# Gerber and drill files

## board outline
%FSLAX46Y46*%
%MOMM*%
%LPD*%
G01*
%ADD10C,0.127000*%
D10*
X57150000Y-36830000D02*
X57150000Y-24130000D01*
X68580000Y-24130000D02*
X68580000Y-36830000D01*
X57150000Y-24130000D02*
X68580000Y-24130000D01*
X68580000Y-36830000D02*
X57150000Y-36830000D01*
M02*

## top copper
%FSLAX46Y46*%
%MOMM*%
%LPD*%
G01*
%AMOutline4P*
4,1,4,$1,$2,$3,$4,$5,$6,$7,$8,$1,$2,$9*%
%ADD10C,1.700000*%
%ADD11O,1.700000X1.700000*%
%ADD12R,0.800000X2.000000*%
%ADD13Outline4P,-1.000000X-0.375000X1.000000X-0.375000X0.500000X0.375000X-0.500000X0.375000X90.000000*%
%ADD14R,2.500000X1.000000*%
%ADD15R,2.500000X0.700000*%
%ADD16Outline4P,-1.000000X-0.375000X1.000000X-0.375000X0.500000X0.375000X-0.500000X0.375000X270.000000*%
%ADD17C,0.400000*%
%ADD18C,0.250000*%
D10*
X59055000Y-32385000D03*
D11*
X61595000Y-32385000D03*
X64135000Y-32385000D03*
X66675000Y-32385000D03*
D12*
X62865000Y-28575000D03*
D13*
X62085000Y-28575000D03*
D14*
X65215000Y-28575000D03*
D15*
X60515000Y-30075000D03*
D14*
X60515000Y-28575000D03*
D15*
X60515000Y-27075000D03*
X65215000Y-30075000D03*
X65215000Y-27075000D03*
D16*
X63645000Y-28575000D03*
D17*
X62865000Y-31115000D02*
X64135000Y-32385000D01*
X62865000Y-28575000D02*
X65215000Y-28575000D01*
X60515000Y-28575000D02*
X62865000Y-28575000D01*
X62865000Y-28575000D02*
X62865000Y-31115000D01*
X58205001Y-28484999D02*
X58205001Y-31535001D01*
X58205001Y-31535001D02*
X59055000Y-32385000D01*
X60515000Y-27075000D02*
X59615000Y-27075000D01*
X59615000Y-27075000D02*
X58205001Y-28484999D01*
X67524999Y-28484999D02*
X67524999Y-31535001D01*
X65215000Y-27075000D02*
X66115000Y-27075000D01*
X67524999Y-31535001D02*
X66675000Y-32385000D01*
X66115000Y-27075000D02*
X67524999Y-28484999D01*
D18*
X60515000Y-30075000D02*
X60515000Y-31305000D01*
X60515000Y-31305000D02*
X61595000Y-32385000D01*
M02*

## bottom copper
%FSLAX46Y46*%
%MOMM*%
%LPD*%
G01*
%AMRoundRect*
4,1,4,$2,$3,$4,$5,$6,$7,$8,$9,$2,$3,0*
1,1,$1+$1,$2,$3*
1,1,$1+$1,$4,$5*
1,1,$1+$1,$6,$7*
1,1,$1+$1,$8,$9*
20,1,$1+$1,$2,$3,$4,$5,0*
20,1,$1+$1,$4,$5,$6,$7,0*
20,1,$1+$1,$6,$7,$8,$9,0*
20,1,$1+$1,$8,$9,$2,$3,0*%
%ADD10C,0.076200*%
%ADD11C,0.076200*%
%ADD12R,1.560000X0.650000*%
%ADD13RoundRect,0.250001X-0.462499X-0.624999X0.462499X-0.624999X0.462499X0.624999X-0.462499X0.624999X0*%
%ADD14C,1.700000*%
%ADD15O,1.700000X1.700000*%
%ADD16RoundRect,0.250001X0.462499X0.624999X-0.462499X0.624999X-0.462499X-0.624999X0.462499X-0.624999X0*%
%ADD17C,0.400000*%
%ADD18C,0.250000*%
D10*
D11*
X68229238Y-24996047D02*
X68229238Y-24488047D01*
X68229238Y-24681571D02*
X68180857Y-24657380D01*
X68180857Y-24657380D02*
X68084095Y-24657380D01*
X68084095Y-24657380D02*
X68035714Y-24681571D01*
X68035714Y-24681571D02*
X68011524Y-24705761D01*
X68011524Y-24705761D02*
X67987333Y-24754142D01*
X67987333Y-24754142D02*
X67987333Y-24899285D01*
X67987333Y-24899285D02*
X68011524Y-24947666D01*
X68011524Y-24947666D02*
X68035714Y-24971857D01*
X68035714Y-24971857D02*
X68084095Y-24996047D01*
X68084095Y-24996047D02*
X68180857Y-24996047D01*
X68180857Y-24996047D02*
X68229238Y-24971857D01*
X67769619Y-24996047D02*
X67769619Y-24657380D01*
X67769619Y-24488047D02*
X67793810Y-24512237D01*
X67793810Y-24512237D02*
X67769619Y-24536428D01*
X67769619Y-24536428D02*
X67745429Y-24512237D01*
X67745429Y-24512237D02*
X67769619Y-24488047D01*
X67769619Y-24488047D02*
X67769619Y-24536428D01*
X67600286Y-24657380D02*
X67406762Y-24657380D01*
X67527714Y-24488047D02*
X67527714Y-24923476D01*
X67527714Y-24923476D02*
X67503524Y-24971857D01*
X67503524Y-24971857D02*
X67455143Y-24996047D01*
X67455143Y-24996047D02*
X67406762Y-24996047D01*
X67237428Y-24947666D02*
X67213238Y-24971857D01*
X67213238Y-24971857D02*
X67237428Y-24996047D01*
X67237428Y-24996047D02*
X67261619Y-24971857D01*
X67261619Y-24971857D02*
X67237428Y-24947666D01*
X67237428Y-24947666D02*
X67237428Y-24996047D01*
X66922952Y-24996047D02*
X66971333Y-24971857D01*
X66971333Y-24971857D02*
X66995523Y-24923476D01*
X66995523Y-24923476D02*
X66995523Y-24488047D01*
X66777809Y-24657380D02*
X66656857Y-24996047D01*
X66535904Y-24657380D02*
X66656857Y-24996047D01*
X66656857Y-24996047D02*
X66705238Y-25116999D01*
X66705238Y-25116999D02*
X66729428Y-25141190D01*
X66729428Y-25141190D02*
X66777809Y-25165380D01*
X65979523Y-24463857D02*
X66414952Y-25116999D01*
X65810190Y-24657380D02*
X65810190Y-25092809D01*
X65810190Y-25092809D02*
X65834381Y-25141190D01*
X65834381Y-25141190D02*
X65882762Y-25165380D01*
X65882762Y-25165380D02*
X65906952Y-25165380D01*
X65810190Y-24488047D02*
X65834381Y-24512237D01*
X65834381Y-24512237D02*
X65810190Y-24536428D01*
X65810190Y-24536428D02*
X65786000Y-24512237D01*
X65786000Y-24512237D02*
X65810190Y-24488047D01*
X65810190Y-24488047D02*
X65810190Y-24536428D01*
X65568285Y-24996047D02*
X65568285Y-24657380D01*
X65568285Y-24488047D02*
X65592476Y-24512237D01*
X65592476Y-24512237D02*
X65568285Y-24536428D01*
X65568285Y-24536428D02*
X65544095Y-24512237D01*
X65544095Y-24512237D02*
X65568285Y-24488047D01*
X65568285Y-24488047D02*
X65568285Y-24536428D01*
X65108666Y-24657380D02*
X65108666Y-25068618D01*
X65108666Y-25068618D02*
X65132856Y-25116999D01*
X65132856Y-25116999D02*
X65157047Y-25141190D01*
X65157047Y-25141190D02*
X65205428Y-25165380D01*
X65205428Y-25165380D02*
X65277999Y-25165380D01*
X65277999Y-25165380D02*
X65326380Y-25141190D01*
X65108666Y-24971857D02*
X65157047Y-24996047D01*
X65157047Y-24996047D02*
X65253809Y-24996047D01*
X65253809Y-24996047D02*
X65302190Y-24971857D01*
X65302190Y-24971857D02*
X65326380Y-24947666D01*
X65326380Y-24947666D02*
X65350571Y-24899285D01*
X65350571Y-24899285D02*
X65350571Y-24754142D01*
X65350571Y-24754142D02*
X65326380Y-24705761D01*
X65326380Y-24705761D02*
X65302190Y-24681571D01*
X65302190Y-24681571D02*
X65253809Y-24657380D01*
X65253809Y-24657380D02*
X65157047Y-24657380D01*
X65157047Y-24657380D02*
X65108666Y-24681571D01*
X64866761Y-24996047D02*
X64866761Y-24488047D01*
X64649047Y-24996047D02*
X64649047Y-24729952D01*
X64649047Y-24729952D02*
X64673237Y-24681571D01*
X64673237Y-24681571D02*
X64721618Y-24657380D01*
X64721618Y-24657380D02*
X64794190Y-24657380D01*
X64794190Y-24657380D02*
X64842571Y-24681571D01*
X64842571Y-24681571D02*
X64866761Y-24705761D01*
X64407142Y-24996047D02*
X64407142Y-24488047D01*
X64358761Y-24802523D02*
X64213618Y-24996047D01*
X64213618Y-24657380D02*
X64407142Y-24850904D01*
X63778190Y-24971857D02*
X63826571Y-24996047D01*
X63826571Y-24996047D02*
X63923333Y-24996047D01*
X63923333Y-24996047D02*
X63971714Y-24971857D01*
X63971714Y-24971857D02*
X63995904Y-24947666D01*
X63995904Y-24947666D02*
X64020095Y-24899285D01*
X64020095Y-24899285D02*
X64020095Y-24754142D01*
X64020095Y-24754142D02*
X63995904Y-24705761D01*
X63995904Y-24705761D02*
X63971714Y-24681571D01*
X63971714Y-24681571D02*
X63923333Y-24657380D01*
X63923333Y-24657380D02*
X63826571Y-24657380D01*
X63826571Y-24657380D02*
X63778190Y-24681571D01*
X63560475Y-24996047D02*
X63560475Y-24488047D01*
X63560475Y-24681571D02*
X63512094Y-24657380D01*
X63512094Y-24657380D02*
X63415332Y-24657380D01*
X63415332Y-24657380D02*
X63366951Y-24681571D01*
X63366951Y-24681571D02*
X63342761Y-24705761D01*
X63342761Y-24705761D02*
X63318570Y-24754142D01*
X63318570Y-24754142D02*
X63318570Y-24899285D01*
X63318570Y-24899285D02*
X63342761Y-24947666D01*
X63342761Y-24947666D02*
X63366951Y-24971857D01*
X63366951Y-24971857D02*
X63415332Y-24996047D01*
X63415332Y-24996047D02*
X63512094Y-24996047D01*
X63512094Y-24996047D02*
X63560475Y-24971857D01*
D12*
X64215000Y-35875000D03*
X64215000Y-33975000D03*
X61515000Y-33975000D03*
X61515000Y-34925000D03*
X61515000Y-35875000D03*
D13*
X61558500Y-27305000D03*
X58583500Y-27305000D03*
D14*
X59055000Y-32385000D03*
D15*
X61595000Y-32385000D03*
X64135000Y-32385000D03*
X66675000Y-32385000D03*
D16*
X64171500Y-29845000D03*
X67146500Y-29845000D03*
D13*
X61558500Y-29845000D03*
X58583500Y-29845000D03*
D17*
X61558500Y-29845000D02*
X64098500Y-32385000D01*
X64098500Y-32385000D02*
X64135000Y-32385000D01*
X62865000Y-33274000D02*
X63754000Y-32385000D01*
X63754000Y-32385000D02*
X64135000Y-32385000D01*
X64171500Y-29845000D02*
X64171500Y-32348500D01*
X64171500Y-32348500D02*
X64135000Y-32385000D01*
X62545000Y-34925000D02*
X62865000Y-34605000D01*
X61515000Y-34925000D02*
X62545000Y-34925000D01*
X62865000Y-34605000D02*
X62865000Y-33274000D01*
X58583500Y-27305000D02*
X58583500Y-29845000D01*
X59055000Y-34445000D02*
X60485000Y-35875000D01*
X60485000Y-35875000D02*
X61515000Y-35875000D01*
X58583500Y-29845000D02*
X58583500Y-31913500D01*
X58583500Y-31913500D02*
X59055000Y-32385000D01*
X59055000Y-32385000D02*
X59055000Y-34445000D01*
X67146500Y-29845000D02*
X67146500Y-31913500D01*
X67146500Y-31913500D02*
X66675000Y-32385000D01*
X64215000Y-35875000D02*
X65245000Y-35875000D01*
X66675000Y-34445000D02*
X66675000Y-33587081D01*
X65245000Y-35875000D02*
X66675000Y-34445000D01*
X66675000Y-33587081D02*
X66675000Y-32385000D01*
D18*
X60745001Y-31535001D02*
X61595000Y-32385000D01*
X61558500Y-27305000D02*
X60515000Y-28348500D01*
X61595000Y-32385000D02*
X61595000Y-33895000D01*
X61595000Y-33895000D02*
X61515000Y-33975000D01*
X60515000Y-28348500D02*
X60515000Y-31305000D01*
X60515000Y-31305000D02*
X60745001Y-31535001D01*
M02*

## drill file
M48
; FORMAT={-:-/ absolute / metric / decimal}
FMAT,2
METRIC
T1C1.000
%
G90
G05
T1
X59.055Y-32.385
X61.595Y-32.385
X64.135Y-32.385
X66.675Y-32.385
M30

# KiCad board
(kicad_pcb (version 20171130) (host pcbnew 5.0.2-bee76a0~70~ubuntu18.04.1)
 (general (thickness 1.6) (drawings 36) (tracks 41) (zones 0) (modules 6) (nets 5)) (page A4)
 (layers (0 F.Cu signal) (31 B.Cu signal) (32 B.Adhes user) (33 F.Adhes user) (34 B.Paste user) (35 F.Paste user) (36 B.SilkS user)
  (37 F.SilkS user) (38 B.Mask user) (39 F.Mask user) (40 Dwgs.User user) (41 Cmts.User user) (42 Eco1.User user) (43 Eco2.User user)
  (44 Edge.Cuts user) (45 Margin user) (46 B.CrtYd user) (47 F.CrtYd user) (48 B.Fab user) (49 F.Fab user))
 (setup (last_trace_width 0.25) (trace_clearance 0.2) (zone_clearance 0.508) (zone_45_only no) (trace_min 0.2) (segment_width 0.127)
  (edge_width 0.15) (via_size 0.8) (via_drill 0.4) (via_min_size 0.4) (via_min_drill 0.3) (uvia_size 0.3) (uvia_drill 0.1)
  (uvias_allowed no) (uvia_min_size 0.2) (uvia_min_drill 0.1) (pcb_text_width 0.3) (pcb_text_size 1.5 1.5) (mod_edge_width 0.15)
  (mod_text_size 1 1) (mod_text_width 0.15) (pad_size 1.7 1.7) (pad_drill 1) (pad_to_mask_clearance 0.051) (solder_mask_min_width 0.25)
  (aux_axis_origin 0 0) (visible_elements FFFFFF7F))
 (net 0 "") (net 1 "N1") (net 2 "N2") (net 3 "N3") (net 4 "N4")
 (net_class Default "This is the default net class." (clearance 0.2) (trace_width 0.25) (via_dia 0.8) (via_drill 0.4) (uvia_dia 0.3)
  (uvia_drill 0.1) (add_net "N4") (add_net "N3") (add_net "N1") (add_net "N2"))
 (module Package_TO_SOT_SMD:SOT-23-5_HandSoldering (layer B.Cu) (at 62.865 34.925)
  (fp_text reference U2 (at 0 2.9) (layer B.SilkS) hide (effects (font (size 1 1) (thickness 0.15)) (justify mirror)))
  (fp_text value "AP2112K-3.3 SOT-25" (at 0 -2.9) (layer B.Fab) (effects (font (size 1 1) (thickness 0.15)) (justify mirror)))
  (pad 5 smd rect (at 1.35 0.95) (size 1.56 0.65) (layers B.Cu B.Paste B.Mask) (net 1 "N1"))
  (pad 4 smd rect (at 1.35 -0.95) (size 1.56 0.65) (layers B.Cu B.Paste B.Mask))
  (pad 3 smd rect (at -1.35 -0.95) (size 1.56 0.65) (layers B.Cu B.Paste B.Mask) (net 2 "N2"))
  (pad 2 smd rect (at -1.35 0) (size 1.56 0.65) (layers B.Cu B.Paste B.Mask) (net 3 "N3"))
  (pad 1 smd rect (at -1.35 0.95) (size 1.56 0.65) (layers B.Cu B.Paste B.Mask) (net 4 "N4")))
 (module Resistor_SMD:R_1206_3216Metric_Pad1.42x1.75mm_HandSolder (layer B.Cu) (at 60.071 27.305)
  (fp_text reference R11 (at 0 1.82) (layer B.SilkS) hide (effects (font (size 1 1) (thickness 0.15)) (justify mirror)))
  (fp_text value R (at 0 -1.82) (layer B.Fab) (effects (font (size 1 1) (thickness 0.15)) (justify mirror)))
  (pad 2 smd roundrect (at 1.4875 0) (size 1.425 1.75) (layers B.Cu B.Paste B.Mask) (roundrect_rratio 0.175439) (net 2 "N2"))
  (pad 1 smd roundrect (at -1.4875 0) (size 1.425 1.75) (layers B.Cu B.Paste B.Mask) (roundrect_rratio 0.175439) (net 4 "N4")))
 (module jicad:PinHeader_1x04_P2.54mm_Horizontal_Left (layer F.Cu) (at 59.055 32.385 90)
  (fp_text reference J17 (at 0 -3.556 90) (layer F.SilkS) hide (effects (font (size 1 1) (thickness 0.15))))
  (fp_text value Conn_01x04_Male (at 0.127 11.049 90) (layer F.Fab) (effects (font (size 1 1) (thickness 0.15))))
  (pad 1 thru_hole circle (at 0 0 90) (size 1.7 1.7) (drill 1) (layers *.Cu *.Mask) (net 4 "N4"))
  (pad 2 thru_hole oval (at 0 2.54 90) (size 1.7 1.7) (drill 1) (layers *.Cu *.Mask) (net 2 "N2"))
  (pad 3 thru_hole oval (at 0 5.08 90) (size 1.7 1.7) (drill 1) (layers *.Cu *.Mask) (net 3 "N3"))
  (pad 4 thru_hole oval (at 0 7.62 90) (size 1.7 1.7) (drill 1) (layers *.Cu *.Mask) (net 1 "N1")))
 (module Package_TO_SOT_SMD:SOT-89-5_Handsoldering (layer F.Cu) (at 62.865 28.575)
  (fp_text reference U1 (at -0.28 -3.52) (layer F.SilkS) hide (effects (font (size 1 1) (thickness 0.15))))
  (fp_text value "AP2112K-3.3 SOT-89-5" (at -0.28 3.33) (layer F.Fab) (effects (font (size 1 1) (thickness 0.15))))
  (pad 2 smd rect (at 0 0 270) (size 2 0.8) (layers F.Cu F.Paste F.Mask) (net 3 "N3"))
  (pad 2 smd trapezoid (at -0.78 0 90) (size 1.5 0.75) (rect_delta 0 0.5) (layers F.Cu F.Paste F.Mask) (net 3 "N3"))
  (pad 2 smd rect (at 2.35 0 270) (size 1 2.5) (layers F.Cu F.Paste F.Mask) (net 3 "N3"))
  (pad 3 smd rect (at -2.35 1.5 270) (size 0.7 2.5) (layers F.Cu F.Paste F.Mask) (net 2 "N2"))
  (pad 2 smd rect (at -2.35 0 270) (size 1 2.5) (layers F.Cu F.Paste F.Mask) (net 3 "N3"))
  (pad 1 smd rect (at -2.35 -1.5 270) (size 0.7 2.5) (layers F.Cu F.Paste F.Mask) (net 4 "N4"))
  (pad 4 smd rect (at 2.35 1.5 270) (size 0.7 2.5) (layers F.Cu F.Paste F.Mask))
  (pad 5 smd rect (at 2.35 -1.5 270) (size 0.7 2.5) (layers F.Cu F.Paste F.Mask) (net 1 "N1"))
  (pad 2 smd trapezoid (at 0.78 0 270) (size 1.5 0.75) (rect_delta 0 0.5) (layers F.Cu F.Paste F.Mask) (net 3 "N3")))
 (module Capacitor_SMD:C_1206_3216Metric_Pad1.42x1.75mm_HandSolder (layer B.Cu) (at 65.659 29.845 180)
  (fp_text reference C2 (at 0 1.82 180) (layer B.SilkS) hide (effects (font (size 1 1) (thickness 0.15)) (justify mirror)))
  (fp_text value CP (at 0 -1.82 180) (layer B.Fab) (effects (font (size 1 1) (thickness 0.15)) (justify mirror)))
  (pad 2 smd roundrect (at 1.4875 0 180) (size 1.425 1.75) (layers B.Cu B.Paste B.Mask) (roundrect_rratio 0.175439) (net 3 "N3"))
  (pad 1 smd roundrect (at -1.4875 0 180) (size 1.425 1.75) (layers B.Cu B.Paste B.Mask) (roundrect_rratio 0.175439) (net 1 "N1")))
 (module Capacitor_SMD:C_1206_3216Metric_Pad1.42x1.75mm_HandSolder (layer B.Cu) (at 60.071 29.845)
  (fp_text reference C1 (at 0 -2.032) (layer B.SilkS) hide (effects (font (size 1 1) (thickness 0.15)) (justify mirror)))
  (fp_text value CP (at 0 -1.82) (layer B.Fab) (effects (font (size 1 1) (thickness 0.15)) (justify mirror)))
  (pad 2 smd roundrect (at 1.4875 0) (size 1.425 1.75) (layers B.Cu B.Paste B.Mask) (roundrect_rratio 0.175439) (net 3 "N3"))
  (pad 1 smd roundrect (at -1.4875 0) (size 1.425 1.75) (layers B.Cu B.Paste B.Mask) (roundrect_rratio 0.175439) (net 4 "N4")))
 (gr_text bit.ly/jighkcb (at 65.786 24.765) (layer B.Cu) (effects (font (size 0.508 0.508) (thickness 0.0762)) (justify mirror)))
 (gr_line (start 57.15 36.83) (end 57.15 24.13) (layer Edge.Cuts) (width 0.127))
 (gr_line (start 68.58 24.13) (end 68.58 36.83) (layer Edge.Cuts) (width 0.127))
 (gr_line (start 57.15 24.13) (end 68.58 24.13) (layer Edge.Cuts) (width 0.127))
 (gr_line (start 68.58 36.83) (end 57.15 36.83) (layer Edge.Cuts) (width 0.127))
 (segment (start 62.865 31.115) (end 64.135 32.385) (width 0.4) (layer F.Cu) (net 3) (status 20))
 (segment (start 62.865 28.575) (end 65.215 28.575) (width 0.4) (layer F.Cu) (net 3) (status 30))
 (segment (start 60.515 28.575) (end 62.865 28.575) (width 0.4) (layer F.Cu) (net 3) (status 30))
 (segment (start 61.5585 29.845) (end 64.0985 32.385) (width 0.4) (layer B.Cu) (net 3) (status 30))
 (segment (start 64.0985 32.385) (end 64.135 32.385) (width 0.4) (layer B.Cu) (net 3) (status 30))
 (segment (start 62.865 28.575) (end 62.865 31.115) (width 0.4) (layer F.Cu) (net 3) (status 10))
 (segment (start 62.865 33.274) (end 63.754 32.385) (width 0.4) (layer B.Cu) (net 3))
 (segment (start 63.754 32.385) (end 64.135 32.385) (width 0.4) (layer B.Cu) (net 3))
 (segment (start 64.1715 29.845) (end 64.1715 32.3485) (width 0.4) (layer B.Cu) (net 3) (status 30))
 (segment (start 64.1715 32.3485) (end 64.135 32.385) (width 0.4) (layer B.Cu) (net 3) (status 30))
 (segment (start 62.545 34.925) (end 62.865 34.605) (width 0.4) (layer B.Cu) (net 3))
 (segment (start 61.515 34.925) (end 62.545 34.925) (width 0.4) (layer B.Cu) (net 3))
 (segment (start 62.865 34.605) (end 62.865 33.274) (width 0.4) (layer B.Cu) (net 3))
 (segment (start 58.5835 27.305) (end 58.5835 29.845) (width 0.4) (layer B.Cu) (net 4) (status 30))
 (segment (start 59.055 34.445) (end 60.485 35.875) (width 0.4) (layer B.Cu) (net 4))
 (segment (start 60.485 35.875) (end 61.515 35.875) (width 0.4) (layer B.Cu) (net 4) (status 20))
 (segment (start 58.5835 29.845) (end 58.5835 31.9135) (width 0.4) (layer B.Cu) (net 4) (status 30))
 (segment (start 58.5835 31.9135) (end 59.055 32.385) (width 0.4) (layer B.Cu) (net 4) (status 30))
 (segment (start 58.205001 28.484999) (end 58.205001 31.535001) (width 0.4) (layer F.Cu) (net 4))
 (segment (start 58.205001 31.535001) (end 59.055 32.385) (width 0.4) (layer F.Cu) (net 4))
 (segment (start 59.055 32.385) (end 59.055 34.445) (width 0.4) (layer B.Cu) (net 4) (status 10))
 (segment (start 60.515 27.075) (end 59.615 27.075) (width 0.4) (layer F.Cu) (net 4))
 (segment (start 59.615 27.075) (end 58.205001 28.484999) (width 0.4) (layer F.Cu) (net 4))
 (segment (start 67.1465 29.845) (end 67.1465 31.9135) (width 0.4) (layer B.Cu) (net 1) (status 30))
 (segment (start 67.1465 31.9135) (end 66.675 32.385) (width 0.4) (layer B.Cu) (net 1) (status 30))
 (segment (start 67.524999 28.484999) (end 67.524999 31.535001) (width 0.4) (layer F.Cu) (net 1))
 (segment (start 64.215 35.875) (end 65.245 35.875) (width 0.4) (layer B.Cu) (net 1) (status 10))
 (segment (start 66.675 34.445) (end 66.675 33.587081) (width 0.4) (layer B.Cu) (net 1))
 (segment (start 65.245 35.875) (end 66.675 34.445) (width 0.4) (layer B.Cu) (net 1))
 (segment (start 66.675 33.587081) (end 66.675 32.385) (width 0.4) (layer B.Cu) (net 1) (status 20))
 (segment (start 65.215 27.075) (end 66.115 27.075) (width 0.4) (layer F.Cu) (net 1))
 (segment (start 67.524999 31.535001) (end 66.675 32.385) (width 0.4) (layer F.Cu) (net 1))
 (segment (start 66.115 27.075) (end 67.524999 28.484999) (width 0.4) (layer F.Cu) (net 1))
 (segment (start 60.745001 31.535001) (end 61.595 32.385) (width 0.25) (layer B.Cu) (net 2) (status 30))
 (segment (start 61.5585 27.305) (end 60.515 28.3485) (width 0.25) (layer B.Cu) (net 2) (status 10))
 (segment (start 60.515 30.075) (end 60.515 31.305) (width 0.25) (layer F.Cu) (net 2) (status 10))
 (segment (start 60.515 31.305) (end 61.595 32.385) (width 0.25) (layer F.Cu) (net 2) (status 20))
 (segment (start 61.595 32.385) (end 61.595 33.895) (width 0.25) (layer B.Cu) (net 2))
 (segment (start 61.595 33.895) (end 61.515 33.975) (width 0.25) (layer B.Cu) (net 2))
 (segment (start 60.515 28.3485) (end 60.515 31.305) (width 0.25) (layer B.Cu) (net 2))
 (segment (start 60.515 31.305) (end 60.745001 31.535001) (width 0.25) (layer B.Cu) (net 2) (status 20)))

